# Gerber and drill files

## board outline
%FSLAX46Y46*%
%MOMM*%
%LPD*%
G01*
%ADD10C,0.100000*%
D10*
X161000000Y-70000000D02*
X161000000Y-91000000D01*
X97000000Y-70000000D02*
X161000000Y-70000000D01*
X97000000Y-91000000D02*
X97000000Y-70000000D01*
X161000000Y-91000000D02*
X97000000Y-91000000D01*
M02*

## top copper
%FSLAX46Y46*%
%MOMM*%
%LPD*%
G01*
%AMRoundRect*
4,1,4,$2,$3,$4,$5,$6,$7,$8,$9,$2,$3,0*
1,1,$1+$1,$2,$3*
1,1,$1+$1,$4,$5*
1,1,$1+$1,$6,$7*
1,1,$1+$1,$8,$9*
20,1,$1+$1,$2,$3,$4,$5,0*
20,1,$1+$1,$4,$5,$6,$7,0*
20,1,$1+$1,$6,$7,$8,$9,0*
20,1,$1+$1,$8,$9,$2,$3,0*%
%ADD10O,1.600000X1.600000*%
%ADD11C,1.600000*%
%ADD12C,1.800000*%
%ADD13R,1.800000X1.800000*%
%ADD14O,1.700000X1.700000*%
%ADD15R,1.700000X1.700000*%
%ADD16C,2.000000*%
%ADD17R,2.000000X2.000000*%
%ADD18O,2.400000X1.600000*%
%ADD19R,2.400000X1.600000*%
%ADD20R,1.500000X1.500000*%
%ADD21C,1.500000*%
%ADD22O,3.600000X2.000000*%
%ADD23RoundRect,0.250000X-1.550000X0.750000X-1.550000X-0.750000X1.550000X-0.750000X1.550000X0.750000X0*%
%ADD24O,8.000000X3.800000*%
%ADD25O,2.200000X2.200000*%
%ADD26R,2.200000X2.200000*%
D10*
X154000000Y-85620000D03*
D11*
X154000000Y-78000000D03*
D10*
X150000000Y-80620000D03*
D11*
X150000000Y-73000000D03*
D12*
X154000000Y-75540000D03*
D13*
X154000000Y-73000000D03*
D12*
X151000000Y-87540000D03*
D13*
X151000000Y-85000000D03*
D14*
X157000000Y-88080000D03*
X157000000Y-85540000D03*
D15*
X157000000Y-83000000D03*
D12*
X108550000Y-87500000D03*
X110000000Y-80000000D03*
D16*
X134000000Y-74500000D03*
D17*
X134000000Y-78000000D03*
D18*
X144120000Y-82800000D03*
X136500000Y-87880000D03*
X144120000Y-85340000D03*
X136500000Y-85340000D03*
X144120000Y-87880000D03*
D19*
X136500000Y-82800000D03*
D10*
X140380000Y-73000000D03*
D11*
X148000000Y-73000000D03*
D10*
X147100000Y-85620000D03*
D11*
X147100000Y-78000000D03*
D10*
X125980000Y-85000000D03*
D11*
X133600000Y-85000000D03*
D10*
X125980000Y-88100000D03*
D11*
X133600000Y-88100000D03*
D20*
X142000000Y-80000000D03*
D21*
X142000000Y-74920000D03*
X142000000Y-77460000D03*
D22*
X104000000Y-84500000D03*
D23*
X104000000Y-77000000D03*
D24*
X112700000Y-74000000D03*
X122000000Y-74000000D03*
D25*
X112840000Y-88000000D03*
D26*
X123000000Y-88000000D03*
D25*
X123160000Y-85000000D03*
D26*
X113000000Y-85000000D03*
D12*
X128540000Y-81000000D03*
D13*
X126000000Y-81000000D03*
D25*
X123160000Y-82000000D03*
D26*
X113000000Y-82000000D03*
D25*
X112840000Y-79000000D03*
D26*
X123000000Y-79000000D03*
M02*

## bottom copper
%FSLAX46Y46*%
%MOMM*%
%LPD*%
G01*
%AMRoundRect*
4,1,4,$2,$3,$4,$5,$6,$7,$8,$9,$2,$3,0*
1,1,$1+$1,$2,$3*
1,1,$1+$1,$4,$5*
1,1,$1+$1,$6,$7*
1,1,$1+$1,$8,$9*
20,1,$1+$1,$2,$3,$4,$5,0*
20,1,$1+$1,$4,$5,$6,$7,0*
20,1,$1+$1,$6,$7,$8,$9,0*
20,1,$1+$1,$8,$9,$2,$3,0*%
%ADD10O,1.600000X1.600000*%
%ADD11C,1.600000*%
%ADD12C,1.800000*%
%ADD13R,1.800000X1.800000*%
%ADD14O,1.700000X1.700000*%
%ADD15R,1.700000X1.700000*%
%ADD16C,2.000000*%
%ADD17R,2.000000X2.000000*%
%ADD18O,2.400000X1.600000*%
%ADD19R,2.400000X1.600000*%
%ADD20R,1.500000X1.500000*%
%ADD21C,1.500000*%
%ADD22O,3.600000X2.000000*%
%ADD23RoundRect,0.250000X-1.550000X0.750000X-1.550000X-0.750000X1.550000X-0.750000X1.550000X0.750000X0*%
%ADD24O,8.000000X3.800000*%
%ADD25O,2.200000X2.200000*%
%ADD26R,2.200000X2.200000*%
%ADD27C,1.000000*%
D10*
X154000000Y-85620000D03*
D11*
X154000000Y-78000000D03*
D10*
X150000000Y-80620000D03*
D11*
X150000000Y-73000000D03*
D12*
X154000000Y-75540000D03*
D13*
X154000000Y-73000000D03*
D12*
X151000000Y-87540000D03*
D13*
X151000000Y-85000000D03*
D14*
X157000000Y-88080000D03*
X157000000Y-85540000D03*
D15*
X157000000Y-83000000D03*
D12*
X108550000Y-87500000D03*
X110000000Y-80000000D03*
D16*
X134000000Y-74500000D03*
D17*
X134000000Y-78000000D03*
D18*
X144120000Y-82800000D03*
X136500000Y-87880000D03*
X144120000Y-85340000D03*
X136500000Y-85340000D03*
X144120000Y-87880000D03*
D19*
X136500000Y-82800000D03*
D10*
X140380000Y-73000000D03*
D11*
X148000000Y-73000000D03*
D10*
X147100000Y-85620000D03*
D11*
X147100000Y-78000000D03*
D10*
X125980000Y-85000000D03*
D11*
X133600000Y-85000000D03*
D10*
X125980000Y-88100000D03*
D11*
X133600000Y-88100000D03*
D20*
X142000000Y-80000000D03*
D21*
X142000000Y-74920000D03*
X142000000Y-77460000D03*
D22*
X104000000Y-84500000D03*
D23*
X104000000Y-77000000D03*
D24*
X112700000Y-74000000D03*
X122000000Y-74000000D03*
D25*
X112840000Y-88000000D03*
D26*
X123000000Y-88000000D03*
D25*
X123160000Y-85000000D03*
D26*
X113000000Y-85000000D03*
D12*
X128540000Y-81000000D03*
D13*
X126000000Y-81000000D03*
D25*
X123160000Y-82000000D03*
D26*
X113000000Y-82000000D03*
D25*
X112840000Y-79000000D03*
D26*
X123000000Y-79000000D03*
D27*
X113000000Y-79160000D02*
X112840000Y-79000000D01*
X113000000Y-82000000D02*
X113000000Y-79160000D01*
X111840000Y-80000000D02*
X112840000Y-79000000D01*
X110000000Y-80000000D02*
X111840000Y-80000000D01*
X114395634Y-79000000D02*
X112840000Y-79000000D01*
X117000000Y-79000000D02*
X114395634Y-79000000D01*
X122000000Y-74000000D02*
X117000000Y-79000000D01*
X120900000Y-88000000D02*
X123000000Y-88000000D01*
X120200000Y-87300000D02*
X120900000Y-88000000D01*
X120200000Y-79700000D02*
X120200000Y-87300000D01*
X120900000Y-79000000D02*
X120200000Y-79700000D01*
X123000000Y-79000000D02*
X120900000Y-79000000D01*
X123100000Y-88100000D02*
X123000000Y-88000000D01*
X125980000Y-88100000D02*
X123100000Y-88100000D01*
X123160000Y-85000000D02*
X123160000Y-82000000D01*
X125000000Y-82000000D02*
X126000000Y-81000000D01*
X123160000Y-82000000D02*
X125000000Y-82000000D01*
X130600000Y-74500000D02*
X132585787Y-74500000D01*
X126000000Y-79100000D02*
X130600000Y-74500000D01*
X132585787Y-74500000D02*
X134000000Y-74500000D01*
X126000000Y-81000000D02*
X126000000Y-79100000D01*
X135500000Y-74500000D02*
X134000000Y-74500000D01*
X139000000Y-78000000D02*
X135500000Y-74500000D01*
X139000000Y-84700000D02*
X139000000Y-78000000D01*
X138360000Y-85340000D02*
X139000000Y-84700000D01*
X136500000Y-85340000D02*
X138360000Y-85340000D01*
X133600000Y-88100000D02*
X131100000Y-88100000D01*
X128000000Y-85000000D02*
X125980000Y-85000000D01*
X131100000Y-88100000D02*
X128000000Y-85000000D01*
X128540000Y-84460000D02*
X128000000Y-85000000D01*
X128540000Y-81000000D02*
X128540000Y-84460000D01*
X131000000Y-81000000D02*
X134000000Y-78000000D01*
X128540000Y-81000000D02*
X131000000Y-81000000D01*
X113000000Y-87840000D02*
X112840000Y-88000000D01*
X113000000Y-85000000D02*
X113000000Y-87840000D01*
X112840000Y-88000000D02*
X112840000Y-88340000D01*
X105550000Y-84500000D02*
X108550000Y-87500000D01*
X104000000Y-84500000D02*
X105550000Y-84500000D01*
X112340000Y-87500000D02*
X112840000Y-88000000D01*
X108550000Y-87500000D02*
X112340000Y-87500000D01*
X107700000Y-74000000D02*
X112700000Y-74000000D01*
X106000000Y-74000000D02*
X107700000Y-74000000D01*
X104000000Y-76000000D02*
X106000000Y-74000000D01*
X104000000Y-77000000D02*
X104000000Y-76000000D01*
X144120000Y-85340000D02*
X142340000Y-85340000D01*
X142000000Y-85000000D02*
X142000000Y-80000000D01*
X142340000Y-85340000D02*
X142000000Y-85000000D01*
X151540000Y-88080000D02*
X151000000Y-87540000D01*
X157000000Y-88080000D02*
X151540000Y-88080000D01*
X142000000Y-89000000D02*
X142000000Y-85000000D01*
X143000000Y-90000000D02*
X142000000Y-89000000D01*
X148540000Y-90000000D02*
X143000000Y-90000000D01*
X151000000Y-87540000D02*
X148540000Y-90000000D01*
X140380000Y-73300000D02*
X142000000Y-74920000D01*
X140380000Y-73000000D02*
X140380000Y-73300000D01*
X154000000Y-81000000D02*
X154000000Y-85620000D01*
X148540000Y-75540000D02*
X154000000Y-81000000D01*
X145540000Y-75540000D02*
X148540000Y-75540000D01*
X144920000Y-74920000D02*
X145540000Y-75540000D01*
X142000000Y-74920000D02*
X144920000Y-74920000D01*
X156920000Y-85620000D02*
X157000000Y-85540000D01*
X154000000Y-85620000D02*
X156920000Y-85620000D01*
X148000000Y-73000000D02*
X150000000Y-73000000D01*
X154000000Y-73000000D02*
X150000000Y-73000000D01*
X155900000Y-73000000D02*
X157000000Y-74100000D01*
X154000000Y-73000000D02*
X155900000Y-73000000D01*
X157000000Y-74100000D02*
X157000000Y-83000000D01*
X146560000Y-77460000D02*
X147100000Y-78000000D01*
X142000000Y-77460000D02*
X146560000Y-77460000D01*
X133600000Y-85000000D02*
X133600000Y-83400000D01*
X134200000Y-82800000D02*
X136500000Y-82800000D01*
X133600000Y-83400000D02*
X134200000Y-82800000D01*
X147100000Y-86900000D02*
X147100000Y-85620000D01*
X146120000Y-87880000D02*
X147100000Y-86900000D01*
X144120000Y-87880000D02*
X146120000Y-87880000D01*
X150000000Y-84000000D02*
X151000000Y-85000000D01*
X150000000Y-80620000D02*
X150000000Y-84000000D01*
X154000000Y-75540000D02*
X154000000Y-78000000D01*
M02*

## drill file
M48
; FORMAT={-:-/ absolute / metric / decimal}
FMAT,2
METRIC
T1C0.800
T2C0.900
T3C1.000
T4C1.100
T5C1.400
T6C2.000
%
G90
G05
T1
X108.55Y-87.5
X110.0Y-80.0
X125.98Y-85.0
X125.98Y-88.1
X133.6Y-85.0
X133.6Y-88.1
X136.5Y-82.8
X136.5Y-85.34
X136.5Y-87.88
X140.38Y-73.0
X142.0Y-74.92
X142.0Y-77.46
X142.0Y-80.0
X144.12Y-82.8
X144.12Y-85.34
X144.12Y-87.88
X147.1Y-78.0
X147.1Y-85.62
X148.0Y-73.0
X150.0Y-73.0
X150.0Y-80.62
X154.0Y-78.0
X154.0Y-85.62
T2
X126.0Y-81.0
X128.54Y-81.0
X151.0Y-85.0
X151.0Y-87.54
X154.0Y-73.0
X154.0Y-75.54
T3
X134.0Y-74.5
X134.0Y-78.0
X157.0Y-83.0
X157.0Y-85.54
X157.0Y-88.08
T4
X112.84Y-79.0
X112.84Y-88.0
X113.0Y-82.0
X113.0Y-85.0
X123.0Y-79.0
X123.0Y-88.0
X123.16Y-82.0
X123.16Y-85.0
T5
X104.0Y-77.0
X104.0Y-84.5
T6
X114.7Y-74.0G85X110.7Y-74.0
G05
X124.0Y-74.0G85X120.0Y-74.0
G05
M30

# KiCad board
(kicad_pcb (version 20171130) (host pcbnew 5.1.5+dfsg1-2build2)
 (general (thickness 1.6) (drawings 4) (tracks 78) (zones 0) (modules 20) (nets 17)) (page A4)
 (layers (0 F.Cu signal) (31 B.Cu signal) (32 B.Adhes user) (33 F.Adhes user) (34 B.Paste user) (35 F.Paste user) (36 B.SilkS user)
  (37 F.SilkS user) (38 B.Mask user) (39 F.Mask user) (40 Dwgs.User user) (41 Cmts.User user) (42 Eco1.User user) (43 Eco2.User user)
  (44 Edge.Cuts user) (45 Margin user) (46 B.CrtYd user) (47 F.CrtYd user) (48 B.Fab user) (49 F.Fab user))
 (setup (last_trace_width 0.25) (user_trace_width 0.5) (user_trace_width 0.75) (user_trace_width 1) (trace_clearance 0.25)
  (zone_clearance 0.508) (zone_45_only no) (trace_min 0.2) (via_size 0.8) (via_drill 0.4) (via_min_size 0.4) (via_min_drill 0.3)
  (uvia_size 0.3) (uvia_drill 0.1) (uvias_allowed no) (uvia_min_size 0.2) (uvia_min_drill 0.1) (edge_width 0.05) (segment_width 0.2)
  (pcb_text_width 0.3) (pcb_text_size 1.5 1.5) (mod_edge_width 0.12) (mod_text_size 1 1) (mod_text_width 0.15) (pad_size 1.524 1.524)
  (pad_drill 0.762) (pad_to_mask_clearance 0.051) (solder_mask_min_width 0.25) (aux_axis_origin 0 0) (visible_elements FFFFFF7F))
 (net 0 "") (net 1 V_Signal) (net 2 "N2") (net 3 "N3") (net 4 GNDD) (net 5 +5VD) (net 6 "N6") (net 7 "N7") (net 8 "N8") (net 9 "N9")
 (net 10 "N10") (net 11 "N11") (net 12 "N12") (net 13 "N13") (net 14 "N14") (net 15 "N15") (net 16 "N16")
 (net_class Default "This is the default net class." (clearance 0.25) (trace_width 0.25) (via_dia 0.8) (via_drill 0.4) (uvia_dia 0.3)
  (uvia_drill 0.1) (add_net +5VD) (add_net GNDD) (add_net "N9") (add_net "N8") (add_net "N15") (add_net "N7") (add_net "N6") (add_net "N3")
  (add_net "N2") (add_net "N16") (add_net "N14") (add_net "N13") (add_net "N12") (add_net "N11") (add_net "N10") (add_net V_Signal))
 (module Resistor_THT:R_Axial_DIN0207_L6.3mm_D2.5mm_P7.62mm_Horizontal (layer F.Cu) (at 154 78 270)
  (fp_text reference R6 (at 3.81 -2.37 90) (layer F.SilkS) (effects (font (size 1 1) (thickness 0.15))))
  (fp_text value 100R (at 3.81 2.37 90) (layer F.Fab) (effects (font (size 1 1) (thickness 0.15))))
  (pad 2 thru_hole oval (at 7.62 0 270) (size 1.6 1.6) (drill 0.8) (layers *.Cu *.Mask) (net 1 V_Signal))
  (pad 1 thru_hole circle (at 0 0 270) (size 1.6 1.6) (drill 0.8) (layers *.Cu *.Mask) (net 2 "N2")))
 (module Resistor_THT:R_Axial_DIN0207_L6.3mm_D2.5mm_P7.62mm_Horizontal (layer F.Cu) (at 150 73 270)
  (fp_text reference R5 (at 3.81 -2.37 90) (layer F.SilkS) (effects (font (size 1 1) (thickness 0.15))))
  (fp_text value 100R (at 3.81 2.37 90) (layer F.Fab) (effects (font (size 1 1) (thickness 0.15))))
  (pad 2 thru_hole oval (at 7.62 0 270) (size 1.6 1.6) (drill 0.8) (layers *.Cu *.Mask) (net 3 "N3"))
  (pad 1 thru_hole circle (at 0 0 270) (size 1.6 1.6) (drill 0.8) (layers *.Cu *.Mask) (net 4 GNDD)))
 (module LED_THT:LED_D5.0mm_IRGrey (layer F.Cu) (at 154 73 270)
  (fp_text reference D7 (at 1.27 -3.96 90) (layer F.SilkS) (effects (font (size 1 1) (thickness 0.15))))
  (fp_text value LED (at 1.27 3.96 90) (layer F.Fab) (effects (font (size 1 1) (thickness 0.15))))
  (pad 2 thru_hole circle (at 2.54 0 270) (size 1.8 1.8) (drill 0.9) (layers *.Cu *.Mask) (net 2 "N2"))
  (pad 1 thru_hole rect (at 0 0 270) (size 1.8 1.8) (drill 0.9) (layers *.Cu *.Mask) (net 4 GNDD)))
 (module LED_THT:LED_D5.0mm (layer F.Cu) (at 151 85 270)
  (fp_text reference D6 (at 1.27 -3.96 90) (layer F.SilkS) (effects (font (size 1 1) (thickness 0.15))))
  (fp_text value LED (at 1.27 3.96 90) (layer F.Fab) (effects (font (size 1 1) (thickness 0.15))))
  (pad 2 thru_hole circle (at 2.54 0 270) (size 1.8 1.8) (drill 0.9) (layers *.Cu *.Mask) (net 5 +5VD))
  (pad 1 thru_hole rect (at 0 0 270) (size 1.8 1.8) (drill 0.9) (layers *.Cu *.Mask) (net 3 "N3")))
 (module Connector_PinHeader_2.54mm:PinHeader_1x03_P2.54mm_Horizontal (layer F.Cu) (at 157 83)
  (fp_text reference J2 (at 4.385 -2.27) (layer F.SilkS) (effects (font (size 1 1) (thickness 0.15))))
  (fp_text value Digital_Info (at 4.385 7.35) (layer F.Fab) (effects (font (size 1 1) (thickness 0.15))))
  (pad 3 thru_hole oval (at 0 5.08) (size 1.7 1.7) (drill 1) (layers *.Cu *.Mask) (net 5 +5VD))
  (pad 2 thru_hole oval (at 0 2.54) (size 1.7 1.7) (drill 1) (layers *.Cu *.Mask) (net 1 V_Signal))
  (pad 1 thru_hole rect (at 0 0) (size 1.7 1.7) (drill 1) (layers *.Cu *.Mask) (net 4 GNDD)))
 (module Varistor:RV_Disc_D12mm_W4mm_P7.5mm (layer F.Cu) (at 110 80 270)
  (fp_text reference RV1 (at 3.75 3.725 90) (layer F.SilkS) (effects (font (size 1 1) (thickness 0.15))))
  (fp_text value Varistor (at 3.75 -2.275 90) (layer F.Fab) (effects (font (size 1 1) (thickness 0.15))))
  (pad 2 thru_hole circle (at 7.5 1.45 270) (size 1.8 1.8) (drill 0.8) (layers *.Cu *.Mask) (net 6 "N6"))
  (pad 1 thru_hole circle (at 0 0 270) (size 1.8 1.8) (drill 0.8) (layers *.Cu *.Mask) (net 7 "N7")))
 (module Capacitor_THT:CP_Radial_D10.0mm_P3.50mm (layer F.Cu) (at 134 78 90)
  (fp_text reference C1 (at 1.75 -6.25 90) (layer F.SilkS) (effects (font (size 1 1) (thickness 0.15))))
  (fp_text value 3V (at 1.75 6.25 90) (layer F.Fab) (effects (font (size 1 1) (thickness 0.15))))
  (pad 2 thru_hole circle (at 3.5 0 90) (size 2 2) (drill 1) (layers *.Cu *.Mask) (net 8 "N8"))
  (pad 1 thru_hole rect (at 0 0 90) (size 2 2) (drill 1) (layers *.Cu *.Mask) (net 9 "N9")))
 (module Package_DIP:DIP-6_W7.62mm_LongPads (layer F.Cu) (at 136.5 82.8)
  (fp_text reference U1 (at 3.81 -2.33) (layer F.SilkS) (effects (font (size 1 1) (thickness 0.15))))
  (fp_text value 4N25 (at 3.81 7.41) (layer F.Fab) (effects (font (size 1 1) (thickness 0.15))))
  (pad 6 thru_hole oval (at 7.62 0) (size 2.4 1.6) (drill 0.8) (layers *.Cu *.Mask) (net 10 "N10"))
  (pad 3 thru_hole oval (at 0 5.08) (size 2.4 1.6) (drill 0.8) (layers *.Cu *.Mask) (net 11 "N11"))
  (pad 5 thru_hole oval (at 7.62 2.54) (size 2.4 1.6) (drill 0.8) (layers *.Cu *.Mask) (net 5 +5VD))
  (pad 2 thru_hole oval (at 0 2.54) (size 2.4 1.6) (drill 0.8) (layers *.Cu *.Mask) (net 8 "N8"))
  (pad 4 thru_hole oval (at 7.62 5.08) (size 2.4 1.6) (drill 0.8) (layers *.Cu *.Mask) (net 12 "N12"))
  (pad 1 thru_hole rect (at 0 0) (size 2.4 1.6) (drill 0.8) (layers *.Cu *.Mask) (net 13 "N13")))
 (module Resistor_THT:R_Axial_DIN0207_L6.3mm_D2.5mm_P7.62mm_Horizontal (layer F.Cu) (at 148 73 180)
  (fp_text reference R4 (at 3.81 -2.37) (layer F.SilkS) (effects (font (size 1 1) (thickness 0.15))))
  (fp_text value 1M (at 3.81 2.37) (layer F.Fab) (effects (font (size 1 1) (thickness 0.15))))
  (pad 2 thru_hole oval (at 7.62 0 180) (size 1.6 1.6) (drill 0.8) (layers *.Cu *.Mask) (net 1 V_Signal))
  (pad 1 thru_hole circle (at 0 0 180) (size 1.6 1.6) (drill 0.8) (layers *.Cu *.Mask) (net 4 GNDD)))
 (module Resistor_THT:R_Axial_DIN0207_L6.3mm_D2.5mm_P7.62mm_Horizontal (layer F.Cu) (at 147.1 78 270)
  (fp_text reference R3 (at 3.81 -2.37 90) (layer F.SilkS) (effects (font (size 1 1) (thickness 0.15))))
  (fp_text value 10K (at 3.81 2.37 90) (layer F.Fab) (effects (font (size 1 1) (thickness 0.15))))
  (pad 2 thru_hole oval (at 7.62 0 270) (size 1.6 1.6) (drill 0.8) (layers *.Cu *.Mask) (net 12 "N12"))
  (pad 1 thru_hole circle (at 0 0 270) (size 1.6 1.6) (drill 0.8) (layers *.Cu *.Mask) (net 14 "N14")))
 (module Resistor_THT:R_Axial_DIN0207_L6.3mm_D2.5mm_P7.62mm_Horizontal (layer F.Cu) (at 133.6 85 180)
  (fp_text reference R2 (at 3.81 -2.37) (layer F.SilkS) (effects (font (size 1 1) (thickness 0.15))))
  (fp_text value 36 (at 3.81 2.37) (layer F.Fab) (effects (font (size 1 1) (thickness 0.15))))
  (pad 2 thru_hole oval (at 7.62 0 180) (size 1.6 1.6) (drill 0.8) (layers *.Cu *.Mask) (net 9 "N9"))
  (pad 1 thru_hole circle (at 0 0 180) (size 1.6 1.6) (drill 0.8) (layers *.Cu *.Mask) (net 13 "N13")))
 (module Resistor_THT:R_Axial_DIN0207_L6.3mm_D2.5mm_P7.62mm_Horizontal (layer F.Cu) (at 133.6 88.1 180)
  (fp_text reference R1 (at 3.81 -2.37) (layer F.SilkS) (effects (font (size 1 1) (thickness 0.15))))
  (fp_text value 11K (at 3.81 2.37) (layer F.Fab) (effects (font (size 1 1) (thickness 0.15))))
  (pad 2 thru_hole oval (at 7.62 0 180) (size 1.6 1.6) (drill 0.8) (layers *.Cu *.Mask) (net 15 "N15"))
  (pad 1 thru_hole circle (at 0 0 180) (size 1.6 1.6) (drill 0.8) (layers *.Cu *.Mask) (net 9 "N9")))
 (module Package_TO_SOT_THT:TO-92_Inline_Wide (layer F.Cu) (at 142 80 90)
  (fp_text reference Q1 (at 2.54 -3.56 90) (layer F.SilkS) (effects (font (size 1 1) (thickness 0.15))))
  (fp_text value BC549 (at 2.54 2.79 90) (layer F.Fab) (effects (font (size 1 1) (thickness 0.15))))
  (pad 1 thru_hole rect (at 0 0 180) (size 1.5 1.5) (drill 0.8) (layers *.Cu *.Mask) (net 5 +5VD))
  (pad 3 thru_hole circle (at 5.08 0 180) (size 1.5 1.5) (drill 0.8) (layers *.Cu *.Mask) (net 1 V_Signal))
  (pad 2 thru_hole circle (at 2.54 0 180) (size 1.5 1.5) (drill 0.8) (layers *.Cu *.Mask) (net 14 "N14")))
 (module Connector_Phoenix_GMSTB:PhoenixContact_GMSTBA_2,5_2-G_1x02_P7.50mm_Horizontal (layer F.Cu) (at 104 77 270)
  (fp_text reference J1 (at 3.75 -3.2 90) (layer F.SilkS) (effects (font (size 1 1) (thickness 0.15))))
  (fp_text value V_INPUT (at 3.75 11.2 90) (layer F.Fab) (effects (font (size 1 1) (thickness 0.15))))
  (pad 2 thru_hole oval (at 7.5 0 270) (size 2 3.6) (drill 1.4) (layers *.Cu *.Mask) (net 6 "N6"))
  (pad 1 thru_hole roundrect (at 0 0 270) (size 2 3.6) (drill 1.4) (layers *.Cu *.Mask) (roundrect_rratio 0.125) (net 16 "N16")))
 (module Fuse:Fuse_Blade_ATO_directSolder (layer F.Cu) (at 122 74 180)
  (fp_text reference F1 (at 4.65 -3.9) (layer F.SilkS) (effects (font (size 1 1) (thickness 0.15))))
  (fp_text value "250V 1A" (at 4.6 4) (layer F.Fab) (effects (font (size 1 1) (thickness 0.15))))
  (pad 2 thru_hole oval (at 9.3 0 180) (size 8 3.8) (drill oval 6 2) (layers *.Cu *.Mask) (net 16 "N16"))
  (pad 1 thru_hole oval (at 0 0 180) (size 8 3.8) (drill oval 6 2) (layers *.Cu *.Mask) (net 7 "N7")))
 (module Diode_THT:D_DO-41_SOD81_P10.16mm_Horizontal (layer F.Cu) (at 123 88 180)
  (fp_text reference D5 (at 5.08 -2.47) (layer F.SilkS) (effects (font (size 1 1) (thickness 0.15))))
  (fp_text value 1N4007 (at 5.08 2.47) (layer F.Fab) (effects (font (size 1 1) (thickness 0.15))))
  (pad 2 thru_hole oval (at 10.16 0 180) (size 2.2 2.2) (drill 1.1) (layers *.Cu *.Mask) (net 6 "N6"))
  (pad 1 thru_hole rect (at 0 0 180) (size 2.2 2.2) (drill 1.1) (layers *.Cu *.Mask) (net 15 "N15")))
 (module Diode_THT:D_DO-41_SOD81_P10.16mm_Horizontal (layer F.Cu) (at 113 85)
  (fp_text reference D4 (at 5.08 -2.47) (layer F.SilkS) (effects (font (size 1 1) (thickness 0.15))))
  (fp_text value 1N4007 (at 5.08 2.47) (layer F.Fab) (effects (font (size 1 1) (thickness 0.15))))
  (pad 2 thru_hole oval (at 10.16 0) (size 2.2 2.2) (drill 1.1) (layers *.Cu *.Mask) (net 8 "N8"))
  (pad 1 thru_hole rect (at 0 0) (size 2.2 2.2) (drill 1.1) (layers *.Cu *.Mask) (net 6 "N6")))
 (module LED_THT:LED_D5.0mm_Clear (layer F.Cu) (at 126 81)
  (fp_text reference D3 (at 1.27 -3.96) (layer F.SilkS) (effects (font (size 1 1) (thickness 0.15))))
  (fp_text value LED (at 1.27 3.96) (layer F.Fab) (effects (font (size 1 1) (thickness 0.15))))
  (pad 2 thru_hole circle (at 2.54 0) (size 1.8 1.8) (drill 0.9) (layers *.Cu *.Mask) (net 9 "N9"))
  (pad 1 thru_hole rect (at 0 0) (size 1.8 1.8) (drill 0.9) (layers *.Cu *.Mask) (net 8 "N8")))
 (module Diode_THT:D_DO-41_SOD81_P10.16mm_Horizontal (layer F.Cu) (at 113 82)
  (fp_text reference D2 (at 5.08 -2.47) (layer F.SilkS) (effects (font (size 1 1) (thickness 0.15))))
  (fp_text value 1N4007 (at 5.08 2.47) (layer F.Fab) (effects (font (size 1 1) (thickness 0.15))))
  (pad 2 thru_hole oval (at 10.16 0) (size 2.2 2.2) (drill 1.1) (layers *.Cu *.Mask) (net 8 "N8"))
  (pad 1 thru_hole rect (at 0 0) (size 2.2 2.2) (drill 1.1) (layers *.Cu *.Mask) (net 7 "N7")))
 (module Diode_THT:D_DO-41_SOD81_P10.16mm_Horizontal (layer F.Cu) (at 123 79 180)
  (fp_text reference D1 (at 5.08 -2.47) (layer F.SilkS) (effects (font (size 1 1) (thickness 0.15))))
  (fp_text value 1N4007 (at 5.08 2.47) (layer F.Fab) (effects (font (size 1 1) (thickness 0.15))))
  (pad 2 thru_hole oval (at 10.16 0 180) (size 2.2 2.2) (drill 1.1) (layers *.Cu *.Mask) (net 7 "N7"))
  (pad 1 thru_hole rect (at 0 0 180) (size 2.2 2.2) (drill 1.1) (layers *.Cu *.Mask) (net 15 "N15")))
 (gr_line (start 161 70) (end 161 91) (layer Edge.Cuts) (width 0.1))
 (gr_line (start 97 70) (end 161 70) (layer Edge.Cuts) (width 0.1))
 (gr_line (start 97 91) (end 97 70) (layer Edge.Cuts) (width 0.1))
 (gr_line (start 161 91) (end 97 91) (layer Edge.Cuts) (width 0.1))
 (segment (start 113 79.16) (end 112.84 79) (width 1) (layer B.Cu) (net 7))
 (segment (start 113 82) (end 113 79.16) (width 1) (layer B.Cu) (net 7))
 (segment (start 111.84 80) (end 112.84 79) (width 1) (layer B.Cu) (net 7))
 (segment (start 110 80) (end 111.84 80) (width 1) (layer B.Cu) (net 7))
 (segment (start 114.395634 79) (end 112.84 79) (width 1) (layer B.Cu) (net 7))
 (segment (start 117 79) (end 114.395634 79) (width 1) (layer B.Cu) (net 7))
 (segment (start 122 74) (end 117 79) (width 1) (layer B.Cu) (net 7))
 (segment (start 120.9 88) (end 123 88) (width 1) (layer B.Cu) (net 15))
 (segment (start 120.2 87.3) (end 120.9 88) (width 1) (layer B.Cu) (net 15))
 (segment (start 120.2 79.7) (end 120.2 87.3) (width 1) (layer B.Cu) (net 15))
 (segment (start 120.9 79) (end 120.2 79.7) (width 1) (layer B.Cu) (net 15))
 (segment (start 123 79) (end 120.9 79) (width 1) (layer B.Cu) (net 15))
 (segment (start 123.1 88.1) (end 123 88) (width 1) (layer B.Cu) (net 15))
 (segment (start 125.98 88.1) (end 123.1 88.1) (width 1) (layer B.Cu) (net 15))
 (segment (start 123.16 85) (end 123.16 82) (width 1) (layer B.Cu) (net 8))
 (segment (start 125 82) (end 126 81) (width 1) (layer B.Cu) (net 8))
 (segment (start 123.16 82) (end 125 82) (width 1) (layer B.Cu) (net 8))
 (segment (start 130.6 74.5) (end 132.585787 74.5) (width 1) (layer B.Cu) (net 8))
 (segment (start 126 79.1) (end 130.6 74.5) (width 1) (layer B.Cu) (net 8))
 (segment (start 132.585787 74.5) (end 134 74.5) (width 1) (layer B.Cu) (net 8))
 (segment (start 126 81) (end 126 79.1) (width 1) (layer B.Cu) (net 8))
 (segment (start 135.5 74.5) (end 134 74.5) (width 1) (layer B.Cu) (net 8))
 (segment (start 139 78) (end 135.5 74.5) (width 1) (layer B.Cu) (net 8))
 (segment (start 139 84.7) (end 139 78) (width 1) (layer B.Cu) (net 8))
 (segment (start 138.36 85.34) (end 139 84.7) (width 1) (layer B.Cu) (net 8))
 (segment (start 136.5 85.34) (end 138.36 85.34) (width 1) (layer B.Cu) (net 8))
 (segment (start 133.6 88.1) (end 131.1 88.1) (width 1) (layer B.Cu) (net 9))
 (segment (start 128 85) (end 125.98 85) (width 1) (layer B.Cu) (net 9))
 (segment (start 131.1 88.1) (end 128 85) (width 1) (layer B.Cu) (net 9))
 (segment (start 128.54 84.46) (end 128 85) (width 1) (layer B.Cu) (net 9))
 (segment (start 128.54 81) (end 128.54 84.46) (width 1) (layer B.Cu) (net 9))
 (segment (start 131 81) (end 134 78) (width 1) (layer B.Cu) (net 9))
 (segment (start 128.54 81) (end 131 81) (width 1) (layer B.Cu) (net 9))
 (segment (start 113 87.84) (end 112.84 88) (width 1) (layer B.Cu) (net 6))
 (segment (start 113 85) (end 113 87.84) (width 1) (layer B.Cu) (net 6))
 (segment (start 112.84 88) (end 112.84 88.34) (width 1) (layer B.Cu) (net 6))
 (segment (start 105.55 84.5) (end 108.55 87.5) (width 1) (layer B.Cu) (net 6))
 (segment (start 104 84.5) (end 105.55 84.5) (width 1) (layer B.Cu) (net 6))
 (segment (start 112.34 87.5) (end 112.84 88) (width 1) (layer B.Cu) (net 6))
 (segment (start 108.55 87.5) (end 112.34 87.5) (width 1) (layer B.Cu) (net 6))
 (segment (start 107.7 74) (end 112.7 74) (width 1) (layer B.Cu) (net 16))
 (segment (start 106 74) (end 107.7 74) (width 1) (layer B.Cu) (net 16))
 (segment (start 104 76) (end 106 74) (width 1) (layer B.Cu) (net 16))
 (segment (start 104 77) (end 104 76) (width 1) (layer B.Cu) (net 16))
 (segment (start 144.12 85.34) (end 142.34 85.34) (width 1) (layer B.Cu) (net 5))
 (segment (start 142 85) (end 142 80) (width 1) (layer B.Cu) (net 5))
 (segment (start 142.34 85.34) (end 142 85) (width 1) (layer B.Cu) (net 5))
 (segment (start 151.54 88.08) (end 151 87.54) (width 1) (layer B.Cu) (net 5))
 (segment (start 157 88.08) (end 151.54 88.08) (width 1) (layer B.Cu) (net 5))
 (segment (start 142 89) (end 142 85) (width 1) (layer B.Cu) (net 5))
 (segment (start 143 90) (end 142 89) (width 1) (layer B.Cu) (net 5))
 (segment (start 148.54 90) (end 143 90) (width 1) (layer B.Cu) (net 5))
 (segment (start 151 87.54) (end 148.54 90) (width 1) (layer B.Cu) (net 5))
 (segment (start 140.38 73.3) (end 142 74.92) (width 1) (layer B.Cu) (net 1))
 (segment (start 140.38 73) (end 140.38 73.3) (width 1) (layer B.Cu) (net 1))
 (segment (start 154 81) (end 154 85.62) (width 1) (layer B.Cu) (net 1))
 (segment (start 148.54 75.54) (end 154 81) (width 1) (layer B.Cu) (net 1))
 (segment (start 145.54 75.54) (end 148.54 75.54) (width 1) (layer B.Cu) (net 1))
 (segment (start 144.92 74.92) (end 145.54 75.54) (width 1) (layer B.Cu) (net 1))
 (segment (start 142 74.92) (end 144.92 74.92) (width 1) (layer B.Cu) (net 1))
 (segment (start 156.92 85.62) (end 157 85.54) (width 1) (layer B.Cu) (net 1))
 (segment (start 154 85.62) (end 156.92 85.62) (width 1) (layer B.Cu) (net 1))
 (segment (start 148 73) (end 150 73) (width 1) (layer B.Cu) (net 4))
 (segment (start 154 73) (end 150 73) (width 1) (layer B.Cu) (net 4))
 (segment (start 155.9 73) (end 157 74.1) (width 1) (layer B.Cu) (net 4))
 (segment (start 154 73) (end 155.9 73) (width 1) (layer B.Cu) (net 4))
 (segment (start 157 74.1) (end 157 83) (width 1) (layer B.Cu) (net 4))
 (segment (start 146.56 77.46) (end 147.1 78) (width 1) (layer B.Cu) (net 14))
 (segment (start 142 77.46) (end 146.56 77.46) (width 1) (layer B.Cu) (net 14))
 (segment (start 133.6 85) (end 133.6 83.4) (width 1) (layer B.Cu) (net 13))
 (segment (start 134.2 82.8) (end 136.5 82.8) (width 1) (layer B.Cu) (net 13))
 (segment (start 133.6 83.4) (end 134.2 82.8) (width 1) (layer B.Cu) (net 13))
 (segment (start 147.1 86.9) (end 147.1 85.62) (width 1) (layer B.Cu) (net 12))
 (segment (start 146.12 87.88) (end 147.1 86.9) (width 1) (layer B.Cu) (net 12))
 (segment (start 144.12 87.88) (end 146.12 87.88) (width 1) (layer B.Cu) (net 12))
 (segment (start 150 84) (end 151 85) (width 1) (layer B.Cu) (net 3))
 (segment (start 150 80.62) (end 150 84) (width 1) (layer B.Cu) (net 3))
 (segment (start 154 75.54) (end 154 78) (width 1) (layer B.Cu) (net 2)))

